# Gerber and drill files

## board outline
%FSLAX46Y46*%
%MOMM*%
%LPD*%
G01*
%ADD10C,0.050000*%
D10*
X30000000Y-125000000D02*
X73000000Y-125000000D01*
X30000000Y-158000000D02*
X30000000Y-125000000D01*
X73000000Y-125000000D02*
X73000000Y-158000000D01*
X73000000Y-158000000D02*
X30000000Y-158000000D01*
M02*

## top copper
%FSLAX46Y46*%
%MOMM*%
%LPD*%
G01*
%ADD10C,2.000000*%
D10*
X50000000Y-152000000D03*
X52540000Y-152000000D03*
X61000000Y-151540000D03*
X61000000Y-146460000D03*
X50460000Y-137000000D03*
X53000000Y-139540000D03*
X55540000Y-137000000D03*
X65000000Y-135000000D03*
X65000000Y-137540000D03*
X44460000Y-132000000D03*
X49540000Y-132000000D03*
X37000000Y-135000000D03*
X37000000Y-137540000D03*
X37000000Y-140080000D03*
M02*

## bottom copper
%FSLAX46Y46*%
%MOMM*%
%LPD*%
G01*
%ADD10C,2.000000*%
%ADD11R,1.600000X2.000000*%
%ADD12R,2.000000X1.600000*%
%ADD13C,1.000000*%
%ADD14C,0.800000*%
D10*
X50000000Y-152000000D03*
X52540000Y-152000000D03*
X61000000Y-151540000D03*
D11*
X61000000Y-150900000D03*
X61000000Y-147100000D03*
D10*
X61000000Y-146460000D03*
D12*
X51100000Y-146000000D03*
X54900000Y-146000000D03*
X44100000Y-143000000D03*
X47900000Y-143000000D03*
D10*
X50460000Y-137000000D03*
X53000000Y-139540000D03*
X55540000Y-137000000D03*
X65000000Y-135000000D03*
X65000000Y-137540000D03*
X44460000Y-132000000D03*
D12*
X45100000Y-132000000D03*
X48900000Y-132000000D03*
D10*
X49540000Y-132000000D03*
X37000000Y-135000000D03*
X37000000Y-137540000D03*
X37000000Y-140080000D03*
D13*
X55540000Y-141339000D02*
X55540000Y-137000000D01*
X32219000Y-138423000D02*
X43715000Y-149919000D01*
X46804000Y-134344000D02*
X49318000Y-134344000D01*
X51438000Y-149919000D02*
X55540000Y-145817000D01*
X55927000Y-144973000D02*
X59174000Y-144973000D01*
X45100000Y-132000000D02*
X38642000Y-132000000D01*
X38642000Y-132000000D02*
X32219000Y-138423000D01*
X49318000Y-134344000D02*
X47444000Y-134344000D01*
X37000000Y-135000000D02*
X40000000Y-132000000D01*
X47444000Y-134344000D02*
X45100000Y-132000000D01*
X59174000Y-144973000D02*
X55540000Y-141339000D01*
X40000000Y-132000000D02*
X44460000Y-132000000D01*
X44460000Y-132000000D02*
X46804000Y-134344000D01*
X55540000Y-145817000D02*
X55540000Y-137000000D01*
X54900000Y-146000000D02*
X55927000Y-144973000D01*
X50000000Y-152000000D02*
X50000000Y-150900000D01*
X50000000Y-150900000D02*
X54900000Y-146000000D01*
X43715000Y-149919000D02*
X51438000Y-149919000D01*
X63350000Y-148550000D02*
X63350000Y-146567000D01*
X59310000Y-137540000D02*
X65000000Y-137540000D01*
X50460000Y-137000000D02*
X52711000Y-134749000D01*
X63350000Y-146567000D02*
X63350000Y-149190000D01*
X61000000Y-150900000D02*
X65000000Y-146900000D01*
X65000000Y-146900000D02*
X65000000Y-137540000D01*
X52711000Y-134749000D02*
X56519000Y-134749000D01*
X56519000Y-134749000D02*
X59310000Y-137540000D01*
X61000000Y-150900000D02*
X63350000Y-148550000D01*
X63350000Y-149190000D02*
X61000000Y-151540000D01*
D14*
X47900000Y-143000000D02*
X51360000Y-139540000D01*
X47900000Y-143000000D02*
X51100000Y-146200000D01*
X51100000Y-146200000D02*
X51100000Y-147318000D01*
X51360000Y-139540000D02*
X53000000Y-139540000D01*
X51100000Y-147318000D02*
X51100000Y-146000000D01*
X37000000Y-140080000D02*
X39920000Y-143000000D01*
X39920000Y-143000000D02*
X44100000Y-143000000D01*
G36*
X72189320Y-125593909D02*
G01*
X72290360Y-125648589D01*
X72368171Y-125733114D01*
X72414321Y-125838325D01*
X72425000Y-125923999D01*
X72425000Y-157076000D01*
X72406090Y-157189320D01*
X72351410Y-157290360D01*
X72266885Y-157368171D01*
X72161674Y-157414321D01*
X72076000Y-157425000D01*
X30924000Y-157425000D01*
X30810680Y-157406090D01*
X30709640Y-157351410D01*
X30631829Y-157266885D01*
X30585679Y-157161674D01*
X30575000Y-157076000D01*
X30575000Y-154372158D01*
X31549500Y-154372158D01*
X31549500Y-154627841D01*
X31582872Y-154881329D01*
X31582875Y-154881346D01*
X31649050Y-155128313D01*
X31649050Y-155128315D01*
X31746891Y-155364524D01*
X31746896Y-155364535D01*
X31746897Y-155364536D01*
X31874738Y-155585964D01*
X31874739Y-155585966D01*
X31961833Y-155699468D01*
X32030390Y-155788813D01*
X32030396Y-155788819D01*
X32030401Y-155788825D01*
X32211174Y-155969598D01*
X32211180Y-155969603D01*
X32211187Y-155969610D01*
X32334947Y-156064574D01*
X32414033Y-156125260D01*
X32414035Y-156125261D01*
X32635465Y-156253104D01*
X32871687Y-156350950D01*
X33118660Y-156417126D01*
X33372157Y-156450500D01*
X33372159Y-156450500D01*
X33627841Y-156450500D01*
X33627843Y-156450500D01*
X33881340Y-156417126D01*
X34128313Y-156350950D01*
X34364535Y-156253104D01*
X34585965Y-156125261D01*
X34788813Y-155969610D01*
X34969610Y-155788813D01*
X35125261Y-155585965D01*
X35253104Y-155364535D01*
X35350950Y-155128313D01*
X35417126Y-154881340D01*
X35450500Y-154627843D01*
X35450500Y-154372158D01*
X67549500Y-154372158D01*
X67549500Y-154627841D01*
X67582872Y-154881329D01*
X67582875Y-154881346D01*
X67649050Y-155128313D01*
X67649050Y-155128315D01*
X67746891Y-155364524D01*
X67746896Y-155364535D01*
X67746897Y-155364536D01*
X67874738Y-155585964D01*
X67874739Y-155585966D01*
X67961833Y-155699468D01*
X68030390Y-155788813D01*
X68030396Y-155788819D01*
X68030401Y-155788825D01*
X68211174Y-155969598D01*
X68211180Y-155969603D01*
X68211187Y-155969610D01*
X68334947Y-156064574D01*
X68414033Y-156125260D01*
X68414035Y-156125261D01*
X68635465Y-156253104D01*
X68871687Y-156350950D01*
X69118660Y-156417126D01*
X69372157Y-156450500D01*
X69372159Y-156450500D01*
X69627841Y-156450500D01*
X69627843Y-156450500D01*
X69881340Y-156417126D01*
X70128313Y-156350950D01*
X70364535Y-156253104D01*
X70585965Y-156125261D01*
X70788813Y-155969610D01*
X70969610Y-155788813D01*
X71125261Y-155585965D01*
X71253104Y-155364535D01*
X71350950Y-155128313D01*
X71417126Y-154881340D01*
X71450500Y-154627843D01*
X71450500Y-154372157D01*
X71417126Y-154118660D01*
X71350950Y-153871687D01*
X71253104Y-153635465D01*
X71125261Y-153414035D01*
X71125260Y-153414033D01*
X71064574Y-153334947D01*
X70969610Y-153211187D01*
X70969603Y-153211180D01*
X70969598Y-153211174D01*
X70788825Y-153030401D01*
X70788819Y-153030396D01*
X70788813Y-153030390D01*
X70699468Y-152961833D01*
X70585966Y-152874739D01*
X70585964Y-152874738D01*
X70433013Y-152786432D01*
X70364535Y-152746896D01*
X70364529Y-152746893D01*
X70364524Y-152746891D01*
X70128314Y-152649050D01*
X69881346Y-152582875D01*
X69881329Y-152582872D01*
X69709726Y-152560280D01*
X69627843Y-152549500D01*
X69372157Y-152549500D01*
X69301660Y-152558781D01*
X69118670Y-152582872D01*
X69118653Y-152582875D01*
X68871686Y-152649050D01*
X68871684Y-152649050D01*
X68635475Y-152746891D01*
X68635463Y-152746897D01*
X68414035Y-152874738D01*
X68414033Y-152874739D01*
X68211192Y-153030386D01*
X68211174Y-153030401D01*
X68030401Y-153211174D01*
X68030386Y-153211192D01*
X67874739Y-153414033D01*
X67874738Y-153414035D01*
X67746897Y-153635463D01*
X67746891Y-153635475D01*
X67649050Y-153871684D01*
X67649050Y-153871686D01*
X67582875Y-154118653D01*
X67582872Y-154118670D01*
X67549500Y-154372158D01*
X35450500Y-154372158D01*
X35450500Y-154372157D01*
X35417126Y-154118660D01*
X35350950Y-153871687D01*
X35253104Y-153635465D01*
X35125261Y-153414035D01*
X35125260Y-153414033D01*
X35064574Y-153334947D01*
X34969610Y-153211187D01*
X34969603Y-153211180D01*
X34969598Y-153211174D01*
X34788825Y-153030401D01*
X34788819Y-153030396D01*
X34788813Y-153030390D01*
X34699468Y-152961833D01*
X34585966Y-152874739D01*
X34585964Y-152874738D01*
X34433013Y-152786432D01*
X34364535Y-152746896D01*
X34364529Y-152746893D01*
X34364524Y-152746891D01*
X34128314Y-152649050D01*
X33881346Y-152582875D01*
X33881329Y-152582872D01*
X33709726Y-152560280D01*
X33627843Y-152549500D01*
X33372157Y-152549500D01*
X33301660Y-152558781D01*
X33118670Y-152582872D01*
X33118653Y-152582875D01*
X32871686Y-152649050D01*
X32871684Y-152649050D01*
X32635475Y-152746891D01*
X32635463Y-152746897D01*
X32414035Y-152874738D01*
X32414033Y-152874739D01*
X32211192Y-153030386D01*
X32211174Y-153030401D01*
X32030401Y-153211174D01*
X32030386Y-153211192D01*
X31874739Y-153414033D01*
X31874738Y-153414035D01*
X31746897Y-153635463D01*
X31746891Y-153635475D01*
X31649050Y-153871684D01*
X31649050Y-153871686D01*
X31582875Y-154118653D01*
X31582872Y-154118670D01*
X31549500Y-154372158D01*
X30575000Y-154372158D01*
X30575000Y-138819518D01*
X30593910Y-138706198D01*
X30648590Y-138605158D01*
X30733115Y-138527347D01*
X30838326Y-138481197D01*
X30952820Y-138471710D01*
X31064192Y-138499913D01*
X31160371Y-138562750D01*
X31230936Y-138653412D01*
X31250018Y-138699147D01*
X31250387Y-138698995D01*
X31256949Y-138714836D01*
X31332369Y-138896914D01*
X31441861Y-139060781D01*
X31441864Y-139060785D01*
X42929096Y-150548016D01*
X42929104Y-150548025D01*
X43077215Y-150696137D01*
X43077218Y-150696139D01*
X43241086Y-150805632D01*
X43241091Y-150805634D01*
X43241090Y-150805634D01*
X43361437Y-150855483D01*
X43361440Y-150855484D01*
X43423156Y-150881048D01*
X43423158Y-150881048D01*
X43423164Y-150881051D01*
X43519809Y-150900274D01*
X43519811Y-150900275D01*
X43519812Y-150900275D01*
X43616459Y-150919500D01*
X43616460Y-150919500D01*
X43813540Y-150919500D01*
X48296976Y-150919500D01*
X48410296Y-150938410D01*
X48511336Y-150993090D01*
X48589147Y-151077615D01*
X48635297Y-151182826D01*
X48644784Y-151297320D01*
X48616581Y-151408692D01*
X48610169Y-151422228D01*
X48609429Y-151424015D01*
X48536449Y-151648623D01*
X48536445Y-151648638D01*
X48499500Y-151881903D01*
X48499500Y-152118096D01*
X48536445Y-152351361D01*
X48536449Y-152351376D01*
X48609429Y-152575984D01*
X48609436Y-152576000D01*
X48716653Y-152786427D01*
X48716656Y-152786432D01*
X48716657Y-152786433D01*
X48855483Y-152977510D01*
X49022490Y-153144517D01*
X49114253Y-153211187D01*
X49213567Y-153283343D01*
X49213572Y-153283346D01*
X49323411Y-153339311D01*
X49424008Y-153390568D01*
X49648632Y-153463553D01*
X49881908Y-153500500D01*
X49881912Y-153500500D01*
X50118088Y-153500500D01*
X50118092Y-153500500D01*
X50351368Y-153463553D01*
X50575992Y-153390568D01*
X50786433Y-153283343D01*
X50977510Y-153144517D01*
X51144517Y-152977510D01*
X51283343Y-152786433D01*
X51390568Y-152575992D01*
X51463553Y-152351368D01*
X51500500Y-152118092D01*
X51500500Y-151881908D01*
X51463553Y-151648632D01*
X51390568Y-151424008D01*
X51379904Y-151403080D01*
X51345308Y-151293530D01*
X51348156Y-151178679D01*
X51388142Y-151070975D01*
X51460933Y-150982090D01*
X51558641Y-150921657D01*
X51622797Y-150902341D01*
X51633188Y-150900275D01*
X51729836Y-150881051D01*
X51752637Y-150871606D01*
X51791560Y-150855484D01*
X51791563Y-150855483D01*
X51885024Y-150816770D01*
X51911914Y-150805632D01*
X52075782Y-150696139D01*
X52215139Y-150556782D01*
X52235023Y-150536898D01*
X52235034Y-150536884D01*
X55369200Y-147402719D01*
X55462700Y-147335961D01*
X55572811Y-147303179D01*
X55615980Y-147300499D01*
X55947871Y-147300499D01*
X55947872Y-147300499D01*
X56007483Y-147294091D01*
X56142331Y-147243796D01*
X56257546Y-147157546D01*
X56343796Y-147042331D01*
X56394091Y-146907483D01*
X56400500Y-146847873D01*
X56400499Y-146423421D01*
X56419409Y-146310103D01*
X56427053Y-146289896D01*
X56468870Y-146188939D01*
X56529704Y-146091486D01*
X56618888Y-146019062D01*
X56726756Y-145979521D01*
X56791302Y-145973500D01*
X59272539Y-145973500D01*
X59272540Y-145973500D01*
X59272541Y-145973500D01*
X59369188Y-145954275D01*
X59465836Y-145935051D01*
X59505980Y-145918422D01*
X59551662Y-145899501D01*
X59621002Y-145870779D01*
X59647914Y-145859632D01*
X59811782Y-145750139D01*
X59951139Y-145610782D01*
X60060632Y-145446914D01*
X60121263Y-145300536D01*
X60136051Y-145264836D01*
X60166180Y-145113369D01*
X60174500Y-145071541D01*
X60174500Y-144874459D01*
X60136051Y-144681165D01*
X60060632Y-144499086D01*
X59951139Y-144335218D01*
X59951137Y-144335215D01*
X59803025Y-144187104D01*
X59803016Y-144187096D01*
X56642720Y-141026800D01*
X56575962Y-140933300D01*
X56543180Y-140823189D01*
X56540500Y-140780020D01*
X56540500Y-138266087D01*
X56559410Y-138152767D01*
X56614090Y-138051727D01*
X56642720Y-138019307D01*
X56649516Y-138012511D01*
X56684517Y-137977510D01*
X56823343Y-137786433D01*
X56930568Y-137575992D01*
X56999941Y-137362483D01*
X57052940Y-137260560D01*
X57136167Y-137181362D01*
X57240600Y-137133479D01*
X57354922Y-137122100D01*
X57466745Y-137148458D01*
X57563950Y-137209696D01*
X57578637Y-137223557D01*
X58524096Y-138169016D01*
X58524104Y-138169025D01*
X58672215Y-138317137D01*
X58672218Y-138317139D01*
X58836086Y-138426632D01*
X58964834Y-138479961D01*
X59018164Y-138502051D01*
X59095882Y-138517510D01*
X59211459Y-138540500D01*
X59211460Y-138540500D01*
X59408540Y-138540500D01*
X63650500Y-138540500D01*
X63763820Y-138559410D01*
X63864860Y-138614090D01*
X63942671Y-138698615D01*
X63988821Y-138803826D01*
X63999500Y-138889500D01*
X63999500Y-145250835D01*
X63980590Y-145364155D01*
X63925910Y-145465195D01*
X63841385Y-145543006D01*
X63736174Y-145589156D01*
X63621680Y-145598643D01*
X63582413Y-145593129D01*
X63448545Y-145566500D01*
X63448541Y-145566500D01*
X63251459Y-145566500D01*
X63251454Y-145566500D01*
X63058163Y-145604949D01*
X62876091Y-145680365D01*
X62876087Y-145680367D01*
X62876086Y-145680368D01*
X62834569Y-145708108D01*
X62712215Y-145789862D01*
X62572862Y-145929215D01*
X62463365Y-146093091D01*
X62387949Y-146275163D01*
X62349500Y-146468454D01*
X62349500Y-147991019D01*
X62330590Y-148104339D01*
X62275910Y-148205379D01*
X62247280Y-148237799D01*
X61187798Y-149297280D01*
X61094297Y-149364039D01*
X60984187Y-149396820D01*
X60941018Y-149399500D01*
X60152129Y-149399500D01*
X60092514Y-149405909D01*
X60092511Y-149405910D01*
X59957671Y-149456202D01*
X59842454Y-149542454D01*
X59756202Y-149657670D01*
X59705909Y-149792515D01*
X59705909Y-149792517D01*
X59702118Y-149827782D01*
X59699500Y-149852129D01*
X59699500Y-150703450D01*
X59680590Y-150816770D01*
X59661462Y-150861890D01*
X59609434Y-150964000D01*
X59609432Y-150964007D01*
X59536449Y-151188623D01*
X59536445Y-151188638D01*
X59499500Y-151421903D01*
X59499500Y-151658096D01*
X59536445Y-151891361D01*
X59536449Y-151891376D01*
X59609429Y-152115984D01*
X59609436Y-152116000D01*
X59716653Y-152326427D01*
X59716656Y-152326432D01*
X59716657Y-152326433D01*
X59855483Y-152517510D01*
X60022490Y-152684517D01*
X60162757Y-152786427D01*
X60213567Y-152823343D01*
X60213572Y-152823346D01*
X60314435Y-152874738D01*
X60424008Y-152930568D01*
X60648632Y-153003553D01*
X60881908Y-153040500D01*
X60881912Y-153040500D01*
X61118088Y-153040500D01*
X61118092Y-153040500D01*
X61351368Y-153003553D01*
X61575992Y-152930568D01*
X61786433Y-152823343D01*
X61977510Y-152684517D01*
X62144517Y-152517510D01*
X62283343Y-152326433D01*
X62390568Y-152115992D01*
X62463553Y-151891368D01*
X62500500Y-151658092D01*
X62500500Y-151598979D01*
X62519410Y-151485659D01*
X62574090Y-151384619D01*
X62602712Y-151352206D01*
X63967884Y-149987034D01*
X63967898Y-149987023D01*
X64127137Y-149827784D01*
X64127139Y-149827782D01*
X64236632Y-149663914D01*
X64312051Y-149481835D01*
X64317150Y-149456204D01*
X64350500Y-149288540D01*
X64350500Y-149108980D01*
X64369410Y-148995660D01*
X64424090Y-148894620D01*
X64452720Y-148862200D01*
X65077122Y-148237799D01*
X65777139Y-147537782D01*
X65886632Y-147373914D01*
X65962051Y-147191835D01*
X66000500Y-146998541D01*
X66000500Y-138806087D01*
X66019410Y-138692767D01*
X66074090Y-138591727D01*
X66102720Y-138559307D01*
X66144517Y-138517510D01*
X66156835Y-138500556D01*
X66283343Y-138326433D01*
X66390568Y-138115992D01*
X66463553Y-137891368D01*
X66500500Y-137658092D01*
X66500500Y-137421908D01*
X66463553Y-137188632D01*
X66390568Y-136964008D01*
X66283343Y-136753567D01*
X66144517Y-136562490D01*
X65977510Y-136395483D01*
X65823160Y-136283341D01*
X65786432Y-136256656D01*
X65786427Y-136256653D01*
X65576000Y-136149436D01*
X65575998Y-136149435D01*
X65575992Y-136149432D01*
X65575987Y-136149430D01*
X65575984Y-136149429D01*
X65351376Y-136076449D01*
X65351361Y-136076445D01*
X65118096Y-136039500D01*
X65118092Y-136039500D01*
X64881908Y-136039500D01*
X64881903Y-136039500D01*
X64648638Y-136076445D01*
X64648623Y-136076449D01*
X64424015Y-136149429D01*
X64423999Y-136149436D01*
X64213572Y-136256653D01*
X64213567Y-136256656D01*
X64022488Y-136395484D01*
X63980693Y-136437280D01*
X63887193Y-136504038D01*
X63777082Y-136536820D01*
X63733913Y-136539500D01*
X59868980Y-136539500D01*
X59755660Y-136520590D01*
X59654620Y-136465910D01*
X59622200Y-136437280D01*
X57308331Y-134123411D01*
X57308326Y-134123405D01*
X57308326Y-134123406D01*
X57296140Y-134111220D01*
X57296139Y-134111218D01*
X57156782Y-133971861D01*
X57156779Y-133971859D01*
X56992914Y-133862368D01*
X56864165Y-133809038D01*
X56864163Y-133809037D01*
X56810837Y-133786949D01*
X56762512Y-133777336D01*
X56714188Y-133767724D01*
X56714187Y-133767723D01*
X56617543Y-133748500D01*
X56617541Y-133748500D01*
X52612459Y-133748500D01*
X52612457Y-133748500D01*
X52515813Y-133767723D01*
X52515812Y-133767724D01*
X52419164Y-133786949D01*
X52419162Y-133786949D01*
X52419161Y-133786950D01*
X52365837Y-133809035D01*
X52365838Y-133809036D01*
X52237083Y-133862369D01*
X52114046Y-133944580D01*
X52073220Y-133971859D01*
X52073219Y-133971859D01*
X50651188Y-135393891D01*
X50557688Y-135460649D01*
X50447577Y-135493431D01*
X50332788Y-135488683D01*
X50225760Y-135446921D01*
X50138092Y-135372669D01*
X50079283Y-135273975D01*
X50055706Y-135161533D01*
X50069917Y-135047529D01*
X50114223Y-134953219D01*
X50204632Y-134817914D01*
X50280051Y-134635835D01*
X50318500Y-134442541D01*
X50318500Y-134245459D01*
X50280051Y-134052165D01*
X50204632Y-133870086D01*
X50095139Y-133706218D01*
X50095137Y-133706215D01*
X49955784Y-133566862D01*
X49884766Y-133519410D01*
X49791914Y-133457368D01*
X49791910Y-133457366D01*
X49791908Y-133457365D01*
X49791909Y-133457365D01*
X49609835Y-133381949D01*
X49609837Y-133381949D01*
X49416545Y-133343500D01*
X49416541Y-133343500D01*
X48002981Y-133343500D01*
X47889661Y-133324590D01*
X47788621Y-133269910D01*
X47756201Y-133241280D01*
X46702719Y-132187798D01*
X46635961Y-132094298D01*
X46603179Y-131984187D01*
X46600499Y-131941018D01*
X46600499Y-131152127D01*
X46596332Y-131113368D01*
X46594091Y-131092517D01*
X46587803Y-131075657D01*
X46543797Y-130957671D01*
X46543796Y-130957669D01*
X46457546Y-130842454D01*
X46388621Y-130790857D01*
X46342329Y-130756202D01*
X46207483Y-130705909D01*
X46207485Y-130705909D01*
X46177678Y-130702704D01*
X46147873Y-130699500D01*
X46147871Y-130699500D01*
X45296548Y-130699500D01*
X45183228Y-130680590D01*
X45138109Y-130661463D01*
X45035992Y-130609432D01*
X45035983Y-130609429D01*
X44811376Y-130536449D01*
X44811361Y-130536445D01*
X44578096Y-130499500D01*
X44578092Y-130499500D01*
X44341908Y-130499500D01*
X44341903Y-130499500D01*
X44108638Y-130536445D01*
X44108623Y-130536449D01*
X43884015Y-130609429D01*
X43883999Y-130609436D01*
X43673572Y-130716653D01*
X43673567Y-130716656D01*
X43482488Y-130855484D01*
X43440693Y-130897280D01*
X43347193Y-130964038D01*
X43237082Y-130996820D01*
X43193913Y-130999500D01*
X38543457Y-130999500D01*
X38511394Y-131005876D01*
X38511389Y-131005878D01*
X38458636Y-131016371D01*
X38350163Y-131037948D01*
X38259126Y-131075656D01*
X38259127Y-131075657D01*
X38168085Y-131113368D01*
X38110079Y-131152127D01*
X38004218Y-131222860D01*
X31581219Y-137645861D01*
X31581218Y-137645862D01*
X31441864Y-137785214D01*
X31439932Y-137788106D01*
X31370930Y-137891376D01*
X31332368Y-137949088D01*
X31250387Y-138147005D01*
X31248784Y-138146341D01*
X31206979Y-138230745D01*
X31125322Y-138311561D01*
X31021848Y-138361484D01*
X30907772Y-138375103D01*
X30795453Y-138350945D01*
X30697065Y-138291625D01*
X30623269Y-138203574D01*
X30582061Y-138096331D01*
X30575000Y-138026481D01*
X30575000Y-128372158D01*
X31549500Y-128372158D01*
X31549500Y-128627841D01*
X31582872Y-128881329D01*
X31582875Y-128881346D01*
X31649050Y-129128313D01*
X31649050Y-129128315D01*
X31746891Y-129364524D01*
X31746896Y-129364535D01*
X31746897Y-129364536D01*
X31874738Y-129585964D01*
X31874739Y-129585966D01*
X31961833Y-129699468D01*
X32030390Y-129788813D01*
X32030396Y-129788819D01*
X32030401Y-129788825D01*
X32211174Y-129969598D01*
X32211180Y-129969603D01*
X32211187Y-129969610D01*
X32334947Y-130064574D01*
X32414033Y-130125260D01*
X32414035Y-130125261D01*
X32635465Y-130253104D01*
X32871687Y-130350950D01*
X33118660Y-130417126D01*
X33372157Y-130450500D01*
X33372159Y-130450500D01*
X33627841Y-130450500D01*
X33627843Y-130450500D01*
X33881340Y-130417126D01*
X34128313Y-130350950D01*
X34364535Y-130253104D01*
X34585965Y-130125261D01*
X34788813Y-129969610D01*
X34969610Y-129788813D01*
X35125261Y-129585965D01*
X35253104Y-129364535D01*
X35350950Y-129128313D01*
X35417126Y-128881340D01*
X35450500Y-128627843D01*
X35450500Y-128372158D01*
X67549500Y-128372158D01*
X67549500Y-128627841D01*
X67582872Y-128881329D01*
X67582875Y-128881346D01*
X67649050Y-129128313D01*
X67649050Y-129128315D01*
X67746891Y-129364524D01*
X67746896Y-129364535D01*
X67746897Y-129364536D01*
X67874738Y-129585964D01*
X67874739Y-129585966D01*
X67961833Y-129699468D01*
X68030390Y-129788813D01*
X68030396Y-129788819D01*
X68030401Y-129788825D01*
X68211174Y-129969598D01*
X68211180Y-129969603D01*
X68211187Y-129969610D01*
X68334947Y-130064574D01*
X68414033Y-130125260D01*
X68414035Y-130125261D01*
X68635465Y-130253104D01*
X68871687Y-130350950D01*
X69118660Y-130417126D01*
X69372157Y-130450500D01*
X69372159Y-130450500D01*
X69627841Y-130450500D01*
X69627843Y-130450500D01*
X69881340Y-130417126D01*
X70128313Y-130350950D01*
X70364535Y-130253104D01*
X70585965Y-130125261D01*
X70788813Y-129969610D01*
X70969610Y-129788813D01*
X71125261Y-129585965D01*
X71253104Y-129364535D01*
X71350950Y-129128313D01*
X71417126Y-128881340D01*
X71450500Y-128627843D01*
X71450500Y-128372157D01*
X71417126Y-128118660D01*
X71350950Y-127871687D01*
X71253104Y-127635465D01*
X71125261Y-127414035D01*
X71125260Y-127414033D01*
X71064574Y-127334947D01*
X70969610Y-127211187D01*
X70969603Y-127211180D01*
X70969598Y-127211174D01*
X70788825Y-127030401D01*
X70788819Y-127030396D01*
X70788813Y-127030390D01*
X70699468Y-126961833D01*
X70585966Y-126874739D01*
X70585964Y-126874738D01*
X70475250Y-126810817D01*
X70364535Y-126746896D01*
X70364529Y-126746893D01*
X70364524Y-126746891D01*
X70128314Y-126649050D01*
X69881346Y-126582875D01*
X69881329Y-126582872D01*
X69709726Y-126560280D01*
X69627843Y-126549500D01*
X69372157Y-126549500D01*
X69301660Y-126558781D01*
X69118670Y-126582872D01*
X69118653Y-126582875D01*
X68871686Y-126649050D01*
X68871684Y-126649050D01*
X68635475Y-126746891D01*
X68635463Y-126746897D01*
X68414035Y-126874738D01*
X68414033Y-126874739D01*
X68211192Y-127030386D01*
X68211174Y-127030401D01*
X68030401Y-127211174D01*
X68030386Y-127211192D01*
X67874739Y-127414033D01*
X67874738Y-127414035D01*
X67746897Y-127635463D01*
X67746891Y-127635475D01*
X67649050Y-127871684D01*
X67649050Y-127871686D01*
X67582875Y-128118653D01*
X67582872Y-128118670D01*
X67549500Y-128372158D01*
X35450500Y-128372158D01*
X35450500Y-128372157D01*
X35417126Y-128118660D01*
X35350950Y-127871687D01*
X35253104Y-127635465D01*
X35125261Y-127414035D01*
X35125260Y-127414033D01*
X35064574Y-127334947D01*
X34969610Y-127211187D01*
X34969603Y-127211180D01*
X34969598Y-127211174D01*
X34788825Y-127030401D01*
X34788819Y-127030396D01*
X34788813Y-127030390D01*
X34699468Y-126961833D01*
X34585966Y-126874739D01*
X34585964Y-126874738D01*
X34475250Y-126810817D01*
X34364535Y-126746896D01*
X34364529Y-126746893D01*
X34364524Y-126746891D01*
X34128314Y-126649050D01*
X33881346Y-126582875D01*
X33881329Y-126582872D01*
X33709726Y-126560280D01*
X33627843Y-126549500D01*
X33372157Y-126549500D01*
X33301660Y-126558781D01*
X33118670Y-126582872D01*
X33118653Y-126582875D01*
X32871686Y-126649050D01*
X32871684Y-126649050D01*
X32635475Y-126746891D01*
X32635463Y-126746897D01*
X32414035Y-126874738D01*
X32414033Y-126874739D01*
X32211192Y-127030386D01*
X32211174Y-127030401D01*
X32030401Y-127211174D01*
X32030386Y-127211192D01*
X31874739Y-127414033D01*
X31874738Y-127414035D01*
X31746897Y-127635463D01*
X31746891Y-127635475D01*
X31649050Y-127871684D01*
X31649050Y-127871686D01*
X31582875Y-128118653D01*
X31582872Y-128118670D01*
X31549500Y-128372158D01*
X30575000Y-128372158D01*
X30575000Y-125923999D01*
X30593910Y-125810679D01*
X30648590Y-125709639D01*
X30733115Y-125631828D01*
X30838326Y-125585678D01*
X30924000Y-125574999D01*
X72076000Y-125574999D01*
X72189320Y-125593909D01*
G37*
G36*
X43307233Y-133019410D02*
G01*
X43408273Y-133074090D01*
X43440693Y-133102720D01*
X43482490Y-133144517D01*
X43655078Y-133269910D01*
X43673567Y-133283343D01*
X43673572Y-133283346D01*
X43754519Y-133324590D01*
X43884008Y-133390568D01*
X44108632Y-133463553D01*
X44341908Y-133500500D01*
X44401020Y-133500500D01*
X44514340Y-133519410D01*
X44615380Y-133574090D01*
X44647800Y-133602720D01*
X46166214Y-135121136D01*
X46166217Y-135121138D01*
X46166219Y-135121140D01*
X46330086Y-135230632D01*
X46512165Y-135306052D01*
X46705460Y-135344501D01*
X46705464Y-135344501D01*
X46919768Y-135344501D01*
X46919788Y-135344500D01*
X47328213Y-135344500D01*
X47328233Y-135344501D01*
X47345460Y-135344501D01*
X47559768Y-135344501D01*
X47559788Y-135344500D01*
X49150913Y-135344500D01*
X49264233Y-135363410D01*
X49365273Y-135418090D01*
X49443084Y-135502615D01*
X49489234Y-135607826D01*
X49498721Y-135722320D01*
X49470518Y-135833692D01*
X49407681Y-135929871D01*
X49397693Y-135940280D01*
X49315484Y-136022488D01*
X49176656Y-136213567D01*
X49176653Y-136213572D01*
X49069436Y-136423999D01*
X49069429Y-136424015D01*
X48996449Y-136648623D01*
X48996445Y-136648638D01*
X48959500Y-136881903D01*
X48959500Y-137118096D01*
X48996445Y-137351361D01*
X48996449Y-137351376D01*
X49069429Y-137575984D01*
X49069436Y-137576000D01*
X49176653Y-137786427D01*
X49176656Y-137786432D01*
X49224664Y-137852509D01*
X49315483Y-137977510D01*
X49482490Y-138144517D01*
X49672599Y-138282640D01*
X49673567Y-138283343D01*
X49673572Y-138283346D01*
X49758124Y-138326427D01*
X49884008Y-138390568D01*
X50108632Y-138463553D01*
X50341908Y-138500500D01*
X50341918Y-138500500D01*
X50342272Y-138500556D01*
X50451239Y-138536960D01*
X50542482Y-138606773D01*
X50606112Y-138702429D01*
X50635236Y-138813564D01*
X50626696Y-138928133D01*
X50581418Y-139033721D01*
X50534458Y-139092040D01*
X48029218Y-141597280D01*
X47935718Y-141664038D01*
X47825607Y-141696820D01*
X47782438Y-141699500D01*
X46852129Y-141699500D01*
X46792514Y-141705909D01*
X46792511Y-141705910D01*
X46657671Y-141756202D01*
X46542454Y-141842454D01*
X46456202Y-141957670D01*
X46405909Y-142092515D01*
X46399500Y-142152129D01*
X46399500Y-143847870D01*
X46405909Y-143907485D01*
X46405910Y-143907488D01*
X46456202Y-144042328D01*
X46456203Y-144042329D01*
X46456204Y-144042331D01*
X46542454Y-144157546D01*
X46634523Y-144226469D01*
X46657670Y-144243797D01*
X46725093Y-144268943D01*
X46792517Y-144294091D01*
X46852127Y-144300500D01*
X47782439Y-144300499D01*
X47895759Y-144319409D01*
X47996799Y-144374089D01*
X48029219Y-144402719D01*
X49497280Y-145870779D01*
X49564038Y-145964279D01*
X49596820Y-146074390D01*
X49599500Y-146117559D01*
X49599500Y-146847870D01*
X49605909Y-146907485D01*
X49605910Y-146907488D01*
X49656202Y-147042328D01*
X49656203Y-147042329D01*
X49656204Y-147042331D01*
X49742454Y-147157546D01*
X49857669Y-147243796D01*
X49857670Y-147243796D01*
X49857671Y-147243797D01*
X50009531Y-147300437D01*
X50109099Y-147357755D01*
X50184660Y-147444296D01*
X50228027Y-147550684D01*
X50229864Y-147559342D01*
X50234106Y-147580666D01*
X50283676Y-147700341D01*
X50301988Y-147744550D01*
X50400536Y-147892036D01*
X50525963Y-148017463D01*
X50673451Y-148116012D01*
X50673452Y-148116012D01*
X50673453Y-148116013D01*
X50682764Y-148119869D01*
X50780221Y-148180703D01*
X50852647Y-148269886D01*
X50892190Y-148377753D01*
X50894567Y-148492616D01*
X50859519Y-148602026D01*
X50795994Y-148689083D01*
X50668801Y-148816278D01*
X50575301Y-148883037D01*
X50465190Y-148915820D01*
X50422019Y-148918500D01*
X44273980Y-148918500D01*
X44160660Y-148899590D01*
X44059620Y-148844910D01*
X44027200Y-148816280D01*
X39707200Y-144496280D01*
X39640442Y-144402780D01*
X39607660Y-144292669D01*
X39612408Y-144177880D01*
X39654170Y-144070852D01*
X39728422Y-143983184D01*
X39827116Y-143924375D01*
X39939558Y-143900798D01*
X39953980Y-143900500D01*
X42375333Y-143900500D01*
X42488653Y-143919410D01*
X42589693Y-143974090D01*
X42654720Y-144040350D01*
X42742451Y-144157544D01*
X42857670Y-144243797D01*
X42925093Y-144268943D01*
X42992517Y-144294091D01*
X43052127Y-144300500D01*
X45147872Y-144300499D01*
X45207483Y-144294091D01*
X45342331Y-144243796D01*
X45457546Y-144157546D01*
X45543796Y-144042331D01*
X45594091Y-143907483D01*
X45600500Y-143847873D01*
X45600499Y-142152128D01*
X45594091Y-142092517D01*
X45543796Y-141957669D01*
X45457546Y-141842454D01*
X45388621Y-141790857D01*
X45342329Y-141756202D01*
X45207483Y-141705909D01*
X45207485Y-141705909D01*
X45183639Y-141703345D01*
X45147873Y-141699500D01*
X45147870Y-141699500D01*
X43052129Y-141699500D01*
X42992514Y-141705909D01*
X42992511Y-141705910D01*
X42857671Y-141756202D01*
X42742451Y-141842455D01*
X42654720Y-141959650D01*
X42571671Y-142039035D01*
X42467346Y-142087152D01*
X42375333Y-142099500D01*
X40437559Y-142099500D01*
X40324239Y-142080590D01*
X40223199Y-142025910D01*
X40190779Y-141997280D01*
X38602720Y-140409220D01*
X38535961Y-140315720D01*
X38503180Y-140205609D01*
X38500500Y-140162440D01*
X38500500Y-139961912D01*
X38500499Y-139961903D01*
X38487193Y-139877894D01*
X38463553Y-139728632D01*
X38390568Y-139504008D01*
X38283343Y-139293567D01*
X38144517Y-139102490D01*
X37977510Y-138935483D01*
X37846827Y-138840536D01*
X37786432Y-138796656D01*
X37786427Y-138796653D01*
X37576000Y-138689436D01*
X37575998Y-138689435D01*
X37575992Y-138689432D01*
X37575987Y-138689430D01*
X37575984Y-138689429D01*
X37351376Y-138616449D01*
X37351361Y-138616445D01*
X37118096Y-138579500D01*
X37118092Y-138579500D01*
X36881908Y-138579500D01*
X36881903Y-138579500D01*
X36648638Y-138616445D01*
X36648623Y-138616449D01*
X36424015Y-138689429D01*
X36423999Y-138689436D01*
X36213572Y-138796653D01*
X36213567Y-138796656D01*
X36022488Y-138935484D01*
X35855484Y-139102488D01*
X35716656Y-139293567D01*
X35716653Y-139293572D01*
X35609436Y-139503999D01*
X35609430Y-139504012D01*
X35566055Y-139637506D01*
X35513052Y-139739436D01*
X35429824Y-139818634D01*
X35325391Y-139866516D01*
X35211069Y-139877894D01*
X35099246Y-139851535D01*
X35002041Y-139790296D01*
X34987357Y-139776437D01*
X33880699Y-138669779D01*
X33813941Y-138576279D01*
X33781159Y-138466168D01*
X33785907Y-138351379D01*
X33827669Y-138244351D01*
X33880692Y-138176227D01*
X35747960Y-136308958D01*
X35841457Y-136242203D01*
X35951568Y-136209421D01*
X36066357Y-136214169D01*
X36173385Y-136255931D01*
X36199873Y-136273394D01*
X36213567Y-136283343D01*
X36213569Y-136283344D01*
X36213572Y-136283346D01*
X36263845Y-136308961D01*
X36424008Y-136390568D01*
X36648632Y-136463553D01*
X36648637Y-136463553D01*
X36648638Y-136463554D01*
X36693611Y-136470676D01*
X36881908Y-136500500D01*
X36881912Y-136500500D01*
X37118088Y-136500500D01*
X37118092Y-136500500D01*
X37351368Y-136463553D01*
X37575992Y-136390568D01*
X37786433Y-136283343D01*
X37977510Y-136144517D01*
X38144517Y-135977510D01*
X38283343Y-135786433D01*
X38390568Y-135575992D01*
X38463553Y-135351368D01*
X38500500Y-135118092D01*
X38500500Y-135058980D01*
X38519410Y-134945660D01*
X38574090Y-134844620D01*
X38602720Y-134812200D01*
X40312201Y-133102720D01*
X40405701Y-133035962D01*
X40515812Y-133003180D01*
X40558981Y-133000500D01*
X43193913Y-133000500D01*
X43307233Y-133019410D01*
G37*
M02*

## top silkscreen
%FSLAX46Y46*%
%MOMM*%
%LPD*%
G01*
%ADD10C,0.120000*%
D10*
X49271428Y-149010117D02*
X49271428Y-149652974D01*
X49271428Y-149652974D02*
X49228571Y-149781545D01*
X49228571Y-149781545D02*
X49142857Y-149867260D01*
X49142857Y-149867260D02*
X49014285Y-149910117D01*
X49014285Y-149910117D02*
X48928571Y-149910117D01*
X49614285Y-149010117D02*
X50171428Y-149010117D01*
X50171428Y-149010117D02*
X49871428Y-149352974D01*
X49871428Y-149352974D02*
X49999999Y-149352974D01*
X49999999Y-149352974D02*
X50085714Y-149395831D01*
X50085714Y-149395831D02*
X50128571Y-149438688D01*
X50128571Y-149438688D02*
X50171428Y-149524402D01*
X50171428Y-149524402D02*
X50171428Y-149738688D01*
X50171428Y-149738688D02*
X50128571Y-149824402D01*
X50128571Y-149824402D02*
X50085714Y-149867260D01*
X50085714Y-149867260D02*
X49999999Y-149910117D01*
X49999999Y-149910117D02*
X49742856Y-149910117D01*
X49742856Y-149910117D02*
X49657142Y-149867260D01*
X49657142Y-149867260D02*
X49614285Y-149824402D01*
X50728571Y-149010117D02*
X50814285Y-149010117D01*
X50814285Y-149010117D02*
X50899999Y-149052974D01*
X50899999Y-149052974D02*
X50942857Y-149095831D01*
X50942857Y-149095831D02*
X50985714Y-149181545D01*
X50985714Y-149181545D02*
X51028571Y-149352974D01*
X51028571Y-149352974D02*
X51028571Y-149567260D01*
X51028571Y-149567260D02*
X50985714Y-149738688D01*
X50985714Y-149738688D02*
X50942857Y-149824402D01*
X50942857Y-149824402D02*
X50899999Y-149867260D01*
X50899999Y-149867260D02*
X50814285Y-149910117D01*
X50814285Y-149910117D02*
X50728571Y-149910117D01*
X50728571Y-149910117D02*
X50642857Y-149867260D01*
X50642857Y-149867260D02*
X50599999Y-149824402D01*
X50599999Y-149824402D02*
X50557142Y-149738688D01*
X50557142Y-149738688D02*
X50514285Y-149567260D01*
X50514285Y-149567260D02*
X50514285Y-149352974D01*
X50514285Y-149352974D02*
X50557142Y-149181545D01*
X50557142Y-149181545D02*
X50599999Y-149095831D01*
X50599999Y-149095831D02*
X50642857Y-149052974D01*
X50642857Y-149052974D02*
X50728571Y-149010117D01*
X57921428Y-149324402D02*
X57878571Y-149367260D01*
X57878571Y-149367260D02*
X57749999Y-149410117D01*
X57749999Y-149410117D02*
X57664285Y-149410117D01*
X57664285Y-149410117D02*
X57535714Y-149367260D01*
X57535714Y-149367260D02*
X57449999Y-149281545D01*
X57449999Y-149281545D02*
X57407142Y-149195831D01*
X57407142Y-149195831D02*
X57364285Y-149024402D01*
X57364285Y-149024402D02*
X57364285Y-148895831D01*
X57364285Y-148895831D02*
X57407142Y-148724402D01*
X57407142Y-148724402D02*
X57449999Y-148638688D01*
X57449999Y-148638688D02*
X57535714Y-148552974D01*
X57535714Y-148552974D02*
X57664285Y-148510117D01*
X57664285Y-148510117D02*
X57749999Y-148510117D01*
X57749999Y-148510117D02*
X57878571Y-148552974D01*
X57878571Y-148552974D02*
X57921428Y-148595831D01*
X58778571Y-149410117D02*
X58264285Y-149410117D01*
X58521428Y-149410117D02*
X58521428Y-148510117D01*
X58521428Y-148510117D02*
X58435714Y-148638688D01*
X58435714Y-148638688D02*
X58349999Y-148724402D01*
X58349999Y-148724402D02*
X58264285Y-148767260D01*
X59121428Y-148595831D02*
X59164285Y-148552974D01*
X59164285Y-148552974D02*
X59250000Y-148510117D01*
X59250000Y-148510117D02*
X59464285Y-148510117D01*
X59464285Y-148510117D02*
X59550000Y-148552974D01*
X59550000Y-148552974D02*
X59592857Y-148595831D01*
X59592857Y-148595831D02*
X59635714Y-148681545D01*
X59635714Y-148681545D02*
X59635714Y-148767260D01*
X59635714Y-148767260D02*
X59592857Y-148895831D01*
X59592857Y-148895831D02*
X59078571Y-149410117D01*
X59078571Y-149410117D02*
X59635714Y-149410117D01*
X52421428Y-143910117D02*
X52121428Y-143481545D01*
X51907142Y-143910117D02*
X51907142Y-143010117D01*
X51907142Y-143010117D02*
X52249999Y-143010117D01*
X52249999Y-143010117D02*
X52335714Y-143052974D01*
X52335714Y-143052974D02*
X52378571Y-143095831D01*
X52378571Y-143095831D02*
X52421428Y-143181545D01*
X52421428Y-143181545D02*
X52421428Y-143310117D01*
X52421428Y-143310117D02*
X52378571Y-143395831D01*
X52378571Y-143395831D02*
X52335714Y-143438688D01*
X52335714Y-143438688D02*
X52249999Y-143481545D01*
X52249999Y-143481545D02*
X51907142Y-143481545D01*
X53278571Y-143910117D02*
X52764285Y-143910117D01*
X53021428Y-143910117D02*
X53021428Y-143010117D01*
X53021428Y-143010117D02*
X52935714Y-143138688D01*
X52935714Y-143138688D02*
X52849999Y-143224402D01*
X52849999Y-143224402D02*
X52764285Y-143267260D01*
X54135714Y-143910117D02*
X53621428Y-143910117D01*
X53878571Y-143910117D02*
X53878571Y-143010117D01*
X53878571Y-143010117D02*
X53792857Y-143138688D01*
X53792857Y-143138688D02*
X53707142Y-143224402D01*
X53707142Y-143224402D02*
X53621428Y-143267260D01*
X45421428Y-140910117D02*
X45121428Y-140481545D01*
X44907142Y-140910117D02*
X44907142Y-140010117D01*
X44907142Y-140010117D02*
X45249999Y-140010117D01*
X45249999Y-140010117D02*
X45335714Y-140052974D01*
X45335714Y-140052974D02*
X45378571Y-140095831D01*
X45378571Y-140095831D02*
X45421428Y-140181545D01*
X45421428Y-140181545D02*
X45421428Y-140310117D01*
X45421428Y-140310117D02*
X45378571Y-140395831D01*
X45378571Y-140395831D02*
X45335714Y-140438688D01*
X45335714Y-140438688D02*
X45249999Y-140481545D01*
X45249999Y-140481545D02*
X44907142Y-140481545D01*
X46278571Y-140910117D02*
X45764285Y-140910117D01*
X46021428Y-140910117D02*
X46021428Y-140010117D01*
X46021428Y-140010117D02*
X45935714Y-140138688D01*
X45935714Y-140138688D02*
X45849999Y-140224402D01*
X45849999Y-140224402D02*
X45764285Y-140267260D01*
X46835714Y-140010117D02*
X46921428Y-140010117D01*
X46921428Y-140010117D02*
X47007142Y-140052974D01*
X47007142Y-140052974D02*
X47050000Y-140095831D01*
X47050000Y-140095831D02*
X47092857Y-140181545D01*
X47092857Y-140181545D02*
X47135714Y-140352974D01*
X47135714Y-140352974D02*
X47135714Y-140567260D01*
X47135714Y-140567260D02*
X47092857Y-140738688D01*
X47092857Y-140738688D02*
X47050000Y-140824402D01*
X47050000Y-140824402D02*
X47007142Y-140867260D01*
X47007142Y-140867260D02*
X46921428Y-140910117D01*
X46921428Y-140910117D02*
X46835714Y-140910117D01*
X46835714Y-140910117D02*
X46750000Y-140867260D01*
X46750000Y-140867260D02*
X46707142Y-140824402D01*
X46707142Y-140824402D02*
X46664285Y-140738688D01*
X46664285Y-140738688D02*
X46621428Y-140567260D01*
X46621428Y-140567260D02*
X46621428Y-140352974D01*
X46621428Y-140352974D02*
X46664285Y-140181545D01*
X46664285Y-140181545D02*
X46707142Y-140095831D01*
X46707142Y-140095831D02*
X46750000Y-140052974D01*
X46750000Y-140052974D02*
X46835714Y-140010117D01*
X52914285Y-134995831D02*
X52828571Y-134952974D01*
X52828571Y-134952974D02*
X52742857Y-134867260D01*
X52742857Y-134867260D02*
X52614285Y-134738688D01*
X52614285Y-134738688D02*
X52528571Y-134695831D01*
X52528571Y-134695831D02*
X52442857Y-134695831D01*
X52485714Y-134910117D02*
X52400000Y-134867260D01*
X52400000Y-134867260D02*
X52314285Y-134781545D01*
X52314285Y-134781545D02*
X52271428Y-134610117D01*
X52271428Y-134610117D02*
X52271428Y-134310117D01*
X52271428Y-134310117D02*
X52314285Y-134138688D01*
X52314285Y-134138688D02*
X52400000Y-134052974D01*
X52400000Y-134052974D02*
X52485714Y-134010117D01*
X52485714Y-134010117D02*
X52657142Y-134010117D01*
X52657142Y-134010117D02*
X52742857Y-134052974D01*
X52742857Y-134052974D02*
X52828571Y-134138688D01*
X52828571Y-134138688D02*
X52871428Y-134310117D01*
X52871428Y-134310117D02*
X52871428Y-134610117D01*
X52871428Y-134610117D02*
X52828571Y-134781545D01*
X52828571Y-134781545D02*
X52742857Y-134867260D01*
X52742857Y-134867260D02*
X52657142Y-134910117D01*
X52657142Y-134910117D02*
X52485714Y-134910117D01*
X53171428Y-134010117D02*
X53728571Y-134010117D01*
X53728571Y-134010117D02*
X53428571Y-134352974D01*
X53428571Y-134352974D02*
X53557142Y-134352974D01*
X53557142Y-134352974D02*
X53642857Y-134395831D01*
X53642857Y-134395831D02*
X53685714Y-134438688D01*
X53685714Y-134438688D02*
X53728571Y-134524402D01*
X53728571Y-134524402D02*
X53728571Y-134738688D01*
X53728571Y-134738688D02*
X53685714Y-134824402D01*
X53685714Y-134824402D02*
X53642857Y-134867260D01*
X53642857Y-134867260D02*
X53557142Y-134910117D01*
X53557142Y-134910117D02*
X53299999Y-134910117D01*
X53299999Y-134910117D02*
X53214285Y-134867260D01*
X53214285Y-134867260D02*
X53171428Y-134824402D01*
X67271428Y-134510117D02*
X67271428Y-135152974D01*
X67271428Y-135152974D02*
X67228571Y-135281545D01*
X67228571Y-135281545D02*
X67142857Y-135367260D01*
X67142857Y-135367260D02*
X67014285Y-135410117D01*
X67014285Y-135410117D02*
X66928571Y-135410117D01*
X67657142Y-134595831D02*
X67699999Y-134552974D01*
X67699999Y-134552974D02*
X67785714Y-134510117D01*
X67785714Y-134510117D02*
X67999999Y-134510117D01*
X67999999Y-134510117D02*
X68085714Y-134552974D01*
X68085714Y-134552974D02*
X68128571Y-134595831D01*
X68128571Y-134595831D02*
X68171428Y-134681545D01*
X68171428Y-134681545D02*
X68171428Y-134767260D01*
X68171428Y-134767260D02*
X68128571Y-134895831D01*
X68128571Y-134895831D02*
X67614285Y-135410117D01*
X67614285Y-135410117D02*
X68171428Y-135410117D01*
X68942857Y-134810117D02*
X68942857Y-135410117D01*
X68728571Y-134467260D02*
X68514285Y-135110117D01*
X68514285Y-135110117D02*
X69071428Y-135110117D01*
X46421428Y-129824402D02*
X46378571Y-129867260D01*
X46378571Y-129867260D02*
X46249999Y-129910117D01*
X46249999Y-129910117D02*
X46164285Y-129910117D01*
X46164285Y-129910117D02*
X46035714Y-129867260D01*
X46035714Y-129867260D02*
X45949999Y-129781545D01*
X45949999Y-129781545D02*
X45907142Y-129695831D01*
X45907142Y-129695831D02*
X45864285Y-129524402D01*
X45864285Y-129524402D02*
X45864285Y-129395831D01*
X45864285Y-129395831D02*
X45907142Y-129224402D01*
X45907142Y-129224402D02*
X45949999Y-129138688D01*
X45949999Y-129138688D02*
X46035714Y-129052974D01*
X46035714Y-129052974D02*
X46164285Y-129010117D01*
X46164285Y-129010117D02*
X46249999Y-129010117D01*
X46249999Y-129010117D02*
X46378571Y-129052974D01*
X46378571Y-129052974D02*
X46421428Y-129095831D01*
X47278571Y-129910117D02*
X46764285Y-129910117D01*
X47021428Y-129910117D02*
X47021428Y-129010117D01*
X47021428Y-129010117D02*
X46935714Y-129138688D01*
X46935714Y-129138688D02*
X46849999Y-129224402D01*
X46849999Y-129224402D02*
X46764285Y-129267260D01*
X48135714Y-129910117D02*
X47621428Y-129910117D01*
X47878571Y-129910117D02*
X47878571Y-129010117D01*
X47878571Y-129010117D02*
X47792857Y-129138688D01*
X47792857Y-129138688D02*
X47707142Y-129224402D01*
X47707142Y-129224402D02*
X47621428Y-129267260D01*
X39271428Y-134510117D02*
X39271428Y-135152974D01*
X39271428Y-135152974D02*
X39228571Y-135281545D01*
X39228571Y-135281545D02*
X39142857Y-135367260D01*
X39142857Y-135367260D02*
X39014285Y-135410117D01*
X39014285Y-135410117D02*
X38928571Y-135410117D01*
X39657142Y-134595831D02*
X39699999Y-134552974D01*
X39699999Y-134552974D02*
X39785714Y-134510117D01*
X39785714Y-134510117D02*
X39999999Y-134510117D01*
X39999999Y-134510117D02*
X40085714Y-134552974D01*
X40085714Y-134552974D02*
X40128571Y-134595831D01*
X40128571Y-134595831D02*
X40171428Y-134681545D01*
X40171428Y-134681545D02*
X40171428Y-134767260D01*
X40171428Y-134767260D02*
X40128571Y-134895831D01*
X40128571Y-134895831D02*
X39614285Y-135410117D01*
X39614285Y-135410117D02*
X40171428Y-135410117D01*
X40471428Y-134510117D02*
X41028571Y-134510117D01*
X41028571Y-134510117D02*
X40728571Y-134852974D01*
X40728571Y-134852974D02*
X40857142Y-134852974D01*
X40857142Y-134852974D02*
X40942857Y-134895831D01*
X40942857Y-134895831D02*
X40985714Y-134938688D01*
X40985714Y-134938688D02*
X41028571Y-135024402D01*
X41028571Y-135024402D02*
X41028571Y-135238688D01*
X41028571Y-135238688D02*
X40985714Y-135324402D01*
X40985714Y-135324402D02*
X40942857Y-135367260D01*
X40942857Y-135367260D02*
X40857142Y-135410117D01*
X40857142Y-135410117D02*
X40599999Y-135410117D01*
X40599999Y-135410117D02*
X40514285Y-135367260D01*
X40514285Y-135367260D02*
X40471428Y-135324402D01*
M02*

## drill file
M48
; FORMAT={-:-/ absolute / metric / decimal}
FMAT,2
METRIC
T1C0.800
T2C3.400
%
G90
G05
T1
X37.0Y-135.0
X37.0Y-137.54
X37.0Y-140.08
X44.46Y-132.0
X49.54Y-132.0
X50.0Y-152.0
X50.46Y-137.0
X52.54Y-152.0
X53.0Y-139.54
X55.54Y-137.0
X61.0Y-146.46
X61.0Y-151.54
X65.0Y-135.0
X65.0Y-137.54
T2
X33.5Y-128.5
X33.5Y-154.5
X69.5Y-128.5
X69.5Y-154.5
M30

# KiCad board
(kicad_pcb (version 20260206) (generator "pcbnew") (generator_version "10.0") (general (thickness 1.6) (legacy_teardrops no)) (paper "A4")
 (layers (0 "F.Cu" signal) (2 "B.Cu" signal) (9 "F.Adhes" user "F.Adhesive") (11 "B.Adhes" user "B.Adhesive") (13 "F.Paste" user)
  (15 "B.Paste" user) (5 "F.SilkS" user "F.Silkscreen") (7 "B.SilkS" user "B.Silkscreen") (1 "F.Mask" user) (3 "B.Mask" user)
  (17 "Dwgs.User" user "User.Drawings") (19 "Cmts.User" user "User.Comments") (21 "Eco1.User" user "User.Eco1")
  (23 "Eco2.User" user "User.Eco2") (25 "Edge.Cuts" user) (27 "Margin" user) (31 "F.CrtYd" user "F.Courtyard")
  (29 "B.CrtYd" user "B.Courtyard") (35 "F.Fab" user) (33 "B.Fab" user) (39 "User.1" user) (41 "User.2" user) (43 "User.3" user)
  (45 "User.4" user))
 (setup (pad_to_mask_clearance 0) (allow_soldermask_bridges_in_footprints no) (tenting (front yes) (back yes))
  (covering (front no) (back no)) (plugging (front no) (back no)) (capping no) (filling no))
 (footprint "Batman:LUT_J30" (layer "F.Cu") (at 50 152)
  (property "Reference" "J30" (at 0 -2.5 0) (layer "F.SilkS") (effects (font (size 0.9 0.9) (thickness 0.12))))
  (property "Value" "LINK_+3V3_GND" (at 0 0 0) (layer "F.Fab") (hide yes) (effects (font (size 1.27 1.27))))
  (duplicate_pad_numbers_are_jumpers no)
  (pad "1" thru_hole circle (at 0 0) (size 2 2) (drill 0.8) (layers "*.Cu") (remove_unused_layers no) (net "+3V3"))
  (pad "2" thru_hole circle (at 2.54 0) (size 2 2) (drill 0.8) (layers "*.Cu") (remove_unused_layers no) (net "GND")))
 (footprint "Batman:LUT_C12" (layer "F.Cu") (at 61 149 90)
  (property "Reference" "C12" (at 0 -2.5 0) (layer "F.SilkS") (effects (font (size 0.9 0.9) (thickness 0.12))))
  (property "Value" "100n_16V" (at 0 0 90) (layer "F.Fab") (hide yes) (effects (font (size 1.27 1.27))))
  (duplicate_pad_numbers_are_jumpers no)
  (pad "1" thru_hole circle (at -2.54 0 90) (size 2 2) (drill 0.8) (layers "*.Cu") (remove_unused_layers no) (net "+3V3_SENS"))
  (pad "1" smd rect (at -1.9 0 90) (size 2 1.6) (layers "B.Cu") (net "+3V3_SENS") (thermal_bridge_angle 45))
  (pad "2" smd rect (at 1.9 0 90) (size 2 1.6) (layers "B.Cu") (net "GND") (thermal_bridge_angle 45))
  (pad "2" thru_hole circle (at 2.54 0 90) (size 2 2) (drill 0.8) (layers "*.Cu") (remove_unused_layers no) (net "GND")))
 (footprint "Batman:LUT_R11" (layer "F.Cu") (at 53 146)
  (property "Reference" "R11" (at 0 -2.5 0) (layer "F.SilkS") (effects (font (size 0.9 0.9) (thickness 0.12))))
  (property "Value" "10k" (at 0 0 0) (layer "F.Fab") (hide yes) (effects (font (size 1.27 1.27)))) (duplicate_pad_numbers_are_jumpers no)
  (pad "1" smd rect (at -1.9 0) (size 2 1.6) (layers "B.Cu") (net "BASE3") (thermal_bridge_angle 45))
  (pad "2" smd rect (at 1.9 0) (size 2 1.6) (layers "B.Cu") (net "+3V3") (thermal_bridge_angle 45)))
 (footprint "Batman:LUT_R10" (layer "F.Cu") (at 46 143)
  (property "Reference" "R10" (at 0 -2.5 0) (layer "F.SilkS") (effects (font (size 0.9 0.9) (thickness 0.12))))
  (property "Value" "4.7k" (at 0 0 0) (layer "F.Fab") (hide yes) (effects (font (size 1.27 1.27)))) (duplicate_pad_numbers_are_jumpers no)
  (pad "1" smd rect (at -1.9 0) (size 2 1.6) (layers "B.Cu") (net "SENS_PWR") (thermal_bridge_angle 45))
  (pad "2" smd rect (at 1.9 0) (size 2 1.6) (layers "B.Cu") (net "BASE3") (thermal_bridge_angle 45)))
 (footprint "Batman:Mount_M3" (layer "F.Cu") (at 69.5 128.5)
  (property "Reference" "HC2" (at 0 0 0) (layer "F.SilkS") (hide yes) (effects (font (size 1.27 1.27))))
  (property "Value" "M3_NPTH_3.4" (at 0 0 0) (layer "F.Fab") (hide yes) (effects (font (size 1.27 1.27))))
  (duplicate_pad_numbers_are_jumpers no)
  (pad "" np_thru_hole circle (at 0 0) (size 3.4 3.4) (drill 3.4) (layers "*.Cu")))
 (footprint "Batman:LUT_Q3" (layer "F.Cu") (at 53 137)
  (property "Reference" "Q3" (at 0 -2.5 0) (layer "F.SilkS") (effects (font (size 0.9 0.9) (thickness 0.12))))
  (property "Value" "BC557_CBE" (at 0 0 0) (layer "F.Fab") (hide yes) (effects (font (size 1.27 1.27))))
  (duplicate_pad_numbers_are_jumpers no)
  (pad "1" thru_hole circle (at -2.54 0) (size 2 2) (drill 0.8) (layers "*.Cu") (remove_unused_layers no) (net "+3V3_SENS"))
  (pad "2" thru_hole circle (at 0 2.54) (size 2 2) (drill 0.8) (layers "*.Cu") (remove_unused_layers no) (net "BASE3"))
  (pad "3" thru_hole circle (at 2.54 0) (size 2 2) (drill 0.8) (layers "*.Cu") (remove_unused_layers no) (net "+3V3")))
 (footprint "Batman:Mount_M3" (layer "F.Cu") (at 69.5 154.5)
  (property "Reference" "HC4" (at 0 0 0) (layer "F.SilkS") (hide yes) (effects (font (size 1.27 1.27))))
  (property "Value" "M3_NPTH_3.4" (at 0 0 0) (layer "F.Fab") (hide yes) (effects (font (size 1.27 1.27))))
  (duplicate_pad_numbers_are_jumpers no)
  (pad "" np_thru_hole circle (at 0 0) (size 3.4 3.4) (drill 3.4) (layers "*.Cu")))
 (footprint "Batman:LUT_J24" (layer "F.Cu") (at 65 135 -90)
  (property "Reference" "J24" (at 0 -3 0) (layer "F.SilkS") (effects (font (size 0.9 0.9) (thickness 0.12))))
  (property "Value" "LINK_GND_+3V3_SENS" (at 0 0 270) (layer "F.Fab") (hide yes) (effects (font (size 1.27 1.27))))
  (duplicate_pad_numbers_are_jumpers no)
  (pad "1" thru_hole circle (at 0 0 270) (size 2 2) (drill 0.8) (layers "*.Cu") (remove_unused_layers no) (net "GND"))
  (pad "2" thru_hole circle (at 2.54 0 270) (size 2 2) (drill 0.8) (layers "*.Cu") (remove_unused_layers no) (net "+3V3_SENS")))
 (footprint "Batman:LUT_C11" (layer "F.Cu") (at 47 132)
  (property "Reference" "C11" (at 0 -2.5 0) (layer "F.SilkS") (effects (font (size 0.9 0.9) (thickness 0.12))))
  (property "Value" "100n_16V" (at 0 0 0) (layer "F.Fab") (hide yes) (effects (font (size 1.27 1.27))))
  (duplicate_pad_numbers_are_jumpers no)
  (pad "1" thru_hole circle (at -2.54 0) (size 2 2) (drill 0.8) (layers "*.Cu") (remove_unused_layers no) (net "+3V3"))
  (pad "1" smd rect (at -1.9 0) (size 2 1.6) (layers "B.Cu") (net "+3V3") (thermal_bridge_angle 45))
  (pad "2" smd rect (at 1.9 0) (size 2 1.6) (layers "B.Cu") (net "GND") (thermal_bridge_angle 45))
  (pad "2" thru_hole circle (at 2.54 0) (size 2 2) (drill 0.8) (layers "*.Cu") (remove_unused_layers no) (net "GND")))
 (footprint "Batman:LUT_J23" (layer "F.Cu") (at 37 135 -90)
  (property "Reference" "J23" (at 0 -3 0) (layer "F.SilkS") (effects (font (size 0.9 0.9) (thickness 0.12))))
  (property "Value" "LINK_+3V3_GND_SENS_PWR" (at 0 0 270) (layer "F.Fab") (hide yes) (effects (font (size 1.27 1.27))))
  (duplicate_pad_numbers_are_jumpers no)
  (pad "1" thru_hole circle (at 0 0 270) (size 2 2) (drill 0.8) (layers "*.Cu") (remove_unused_layers no) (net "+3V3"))
  (pad "2" thru_hole circle (at 2.54 0 270) (size 2 2) (drill 0.8) (layers "*.Cu") (remove_unused_layers no) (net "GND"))
  (pad "3" thru_hole circle (at 5.08 0 270) (size 2 2) (drill 0.8) (layers "*.Cu") (remove_unused_layers no) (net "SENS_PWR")))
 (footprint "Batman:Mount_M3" (layer "F.Cu") (at 33.5 128.5)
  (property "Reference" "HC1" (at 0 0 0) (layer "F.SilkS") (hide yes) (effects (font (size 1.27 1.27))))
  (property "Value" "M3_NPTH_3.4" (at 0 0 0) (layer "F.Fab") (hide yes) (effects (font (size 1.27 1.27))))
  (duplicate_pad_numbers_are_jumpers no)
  (pad "" np_thru_hole circle (at 0 0) (size 3.4 3.4) (drill 3.4) (layers "*.Cu")))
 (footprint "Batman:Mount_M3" (layer "F.Cu") (at 33.5 154.5)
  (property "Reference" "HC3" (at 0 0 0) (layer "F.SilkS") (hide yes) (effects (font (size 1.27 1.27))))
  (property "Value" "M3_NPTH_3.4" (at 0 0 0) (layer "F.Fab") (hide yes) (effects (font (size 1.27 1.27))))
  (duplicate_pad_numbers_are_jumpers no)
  (pad "" np_thru_hole circle (at 0 0) (size 3.4 3.4) (drill 3.4) (layers "*.Cu")))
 (gr_line (start 30 125) (end 73 125) (stroke (width 0.05) (type default)) (layer "Edge.Cuts"))
 (gr_line (start 30 158) (end 30 125) (stroke (width 0.05) (type default)) (layer "Edge.Cuts"))
 (gr_line (start 73 125) (end 73 158) (stroke (width 0.05) (type default)) (layer "Edge.Cuts"))
 (gr_line (start 73 158) (end 30 158) (stroke (width 0.05) (type default)) (layer "Edge.Cuts"))
 (segment (start 55.54 141.339) (end 55.54 137) (width 1) (layer "B.Cu") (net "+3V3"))
 (segment (start 32.219 138.423) (end 43.715 149.919) (width 1) (layer "B.Cu") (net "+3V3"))
 (segment (start 46.804 134.344) (end 49.318 134.344) (width 1) (layer "B.Cu") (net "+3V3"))
 (segment (start 51.438 149.919) (end 55.54 145.817) (width 1) (layer "B.Cu") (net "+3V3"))
 (segment (start 55.927 144.973) (end 59.174 144.973) (width 1) (layer "B.Cu") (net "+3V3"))
 (segment (start 45.1 132) (end 38.642 132) (width 1) (layer "B.Cu") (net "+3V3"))
 (segment (start 38.642 132) (end 32.219 138.423) (width 1) (layer "B.Cu") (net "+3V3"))
 (segment (start 49.318 134.344) (end 47.444 134.344) (width 1) (layer "B.Cu") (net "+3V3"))
 (segment (start 37 135) (end 40 132) (width 1) (layer "B.Cu") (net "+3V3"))
 (segment (start 47.444 134.344) (end 45.1 132) (width 1) (layer "B.Cu") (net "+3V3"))
 (segment (start 59.174 144.973) (end 55.54 141.339) (width 1) (layer "B.Cu") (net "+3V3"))
 (segment (start 40 132) (end 44.46 132) (width 1) (layer "B.Cu") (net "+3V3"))
 (segment (start 44.46 132) (end 46.804 134.344) (width 1) (layer "B.Cu") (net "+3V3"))
 (segment (start 55.54 145.817) (end 55.54 137) (width 1) (layer "B.Cu") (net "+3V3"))
 (segment (start 54.9 146) (end 55.927 144.973) (width 1) (layer "B.Cu") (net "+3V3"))
 (segment (start 50 152) (end 50 150.9) (width 1) (layer "B.Cu") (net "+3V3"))
 (segment (start 50 150.9) (end 54.9 146) (width 1) (layer "B.Cu") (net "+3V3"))
 (segment (start 43.715 149.919) (end 51.438 149.919) (width 1) (layer "B.Cu") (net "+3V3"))
 (segment (start 63.35 148.55) (end 63.35 146.567) (width 1) (layer "B.Cu") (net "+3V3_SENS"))
 (segment (start 59.31 137.54) (end 65 137.54) (width 1) (layer "B.Cu") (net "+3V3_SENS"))
 (segment (start 50.46 137) (end 52.711 134.749) (width 1) (layer "B.Cu") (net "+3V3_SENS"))
 (segment (start 63.35 146.567) (end 63.35 149.19) (width 1) (layer "B.Cu") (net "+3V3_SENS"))
 (segment (start 61 150.9) (end 65 146.9) (width 1) (layer "B.Cu") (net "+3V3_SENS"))
 (segment (start 65 146.9) (end 65 137.54) (width 1) (layer "B.Cu") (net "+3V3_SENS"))
 (segment (start 52.711 134.749) (end 56.519 134.749) (width 1) (layer "B.Cu") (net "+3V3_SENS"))
 (segment (start 56.519 134.749) (end 59.31 137.54) (width 1) (layer "B.Cu") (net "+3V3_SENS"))
 (segment (start 61 150.9) (end 63.35 148.55) (width 1) (layer "B.Cu") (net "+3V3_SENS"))
 (segment (start 63.35 149.19) (end 61 151.54) (width 1) (layer "B.Cu") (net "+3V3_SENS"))
 (segment (start 47.9 143) (end 51.36 139.54) (width 0.8) (layer "B.Cu") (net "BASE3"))
 (segment (start 47.9 143) (end 51.1 146.2) (width 0.8) (layer "B.Cu") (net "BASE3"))
 (segment (start 51.1 146.2) (end 51.1 147.318) (width 0.8) (layer "B.Cu") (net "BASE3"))
 (segment (start 51.36 139.54) (end 53 139.54) (width 0.8) (layer "B.Cu") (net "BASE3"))
 (segment (start 51.1 147.318) (end 51.1 146) (width 0.8) (layer "B.Cu") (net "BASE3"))
 (segment (start 37 140.08) (end 39.92 143) (width 0.8) (layer "B.Cu") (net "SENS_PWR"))
 (segment (start 39.92 143) (end 44.1 143) (width 0.8) (layer "B.Cu") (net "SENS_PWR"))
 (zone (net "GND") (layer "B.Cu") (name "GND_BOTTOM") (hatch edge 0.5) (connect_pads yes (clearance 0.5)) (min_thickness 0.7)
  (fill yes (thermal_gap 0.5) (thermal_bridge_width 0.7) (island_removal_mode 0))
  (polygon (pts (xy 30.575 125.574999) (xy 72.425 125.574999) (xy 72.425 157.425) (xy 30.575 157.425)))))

